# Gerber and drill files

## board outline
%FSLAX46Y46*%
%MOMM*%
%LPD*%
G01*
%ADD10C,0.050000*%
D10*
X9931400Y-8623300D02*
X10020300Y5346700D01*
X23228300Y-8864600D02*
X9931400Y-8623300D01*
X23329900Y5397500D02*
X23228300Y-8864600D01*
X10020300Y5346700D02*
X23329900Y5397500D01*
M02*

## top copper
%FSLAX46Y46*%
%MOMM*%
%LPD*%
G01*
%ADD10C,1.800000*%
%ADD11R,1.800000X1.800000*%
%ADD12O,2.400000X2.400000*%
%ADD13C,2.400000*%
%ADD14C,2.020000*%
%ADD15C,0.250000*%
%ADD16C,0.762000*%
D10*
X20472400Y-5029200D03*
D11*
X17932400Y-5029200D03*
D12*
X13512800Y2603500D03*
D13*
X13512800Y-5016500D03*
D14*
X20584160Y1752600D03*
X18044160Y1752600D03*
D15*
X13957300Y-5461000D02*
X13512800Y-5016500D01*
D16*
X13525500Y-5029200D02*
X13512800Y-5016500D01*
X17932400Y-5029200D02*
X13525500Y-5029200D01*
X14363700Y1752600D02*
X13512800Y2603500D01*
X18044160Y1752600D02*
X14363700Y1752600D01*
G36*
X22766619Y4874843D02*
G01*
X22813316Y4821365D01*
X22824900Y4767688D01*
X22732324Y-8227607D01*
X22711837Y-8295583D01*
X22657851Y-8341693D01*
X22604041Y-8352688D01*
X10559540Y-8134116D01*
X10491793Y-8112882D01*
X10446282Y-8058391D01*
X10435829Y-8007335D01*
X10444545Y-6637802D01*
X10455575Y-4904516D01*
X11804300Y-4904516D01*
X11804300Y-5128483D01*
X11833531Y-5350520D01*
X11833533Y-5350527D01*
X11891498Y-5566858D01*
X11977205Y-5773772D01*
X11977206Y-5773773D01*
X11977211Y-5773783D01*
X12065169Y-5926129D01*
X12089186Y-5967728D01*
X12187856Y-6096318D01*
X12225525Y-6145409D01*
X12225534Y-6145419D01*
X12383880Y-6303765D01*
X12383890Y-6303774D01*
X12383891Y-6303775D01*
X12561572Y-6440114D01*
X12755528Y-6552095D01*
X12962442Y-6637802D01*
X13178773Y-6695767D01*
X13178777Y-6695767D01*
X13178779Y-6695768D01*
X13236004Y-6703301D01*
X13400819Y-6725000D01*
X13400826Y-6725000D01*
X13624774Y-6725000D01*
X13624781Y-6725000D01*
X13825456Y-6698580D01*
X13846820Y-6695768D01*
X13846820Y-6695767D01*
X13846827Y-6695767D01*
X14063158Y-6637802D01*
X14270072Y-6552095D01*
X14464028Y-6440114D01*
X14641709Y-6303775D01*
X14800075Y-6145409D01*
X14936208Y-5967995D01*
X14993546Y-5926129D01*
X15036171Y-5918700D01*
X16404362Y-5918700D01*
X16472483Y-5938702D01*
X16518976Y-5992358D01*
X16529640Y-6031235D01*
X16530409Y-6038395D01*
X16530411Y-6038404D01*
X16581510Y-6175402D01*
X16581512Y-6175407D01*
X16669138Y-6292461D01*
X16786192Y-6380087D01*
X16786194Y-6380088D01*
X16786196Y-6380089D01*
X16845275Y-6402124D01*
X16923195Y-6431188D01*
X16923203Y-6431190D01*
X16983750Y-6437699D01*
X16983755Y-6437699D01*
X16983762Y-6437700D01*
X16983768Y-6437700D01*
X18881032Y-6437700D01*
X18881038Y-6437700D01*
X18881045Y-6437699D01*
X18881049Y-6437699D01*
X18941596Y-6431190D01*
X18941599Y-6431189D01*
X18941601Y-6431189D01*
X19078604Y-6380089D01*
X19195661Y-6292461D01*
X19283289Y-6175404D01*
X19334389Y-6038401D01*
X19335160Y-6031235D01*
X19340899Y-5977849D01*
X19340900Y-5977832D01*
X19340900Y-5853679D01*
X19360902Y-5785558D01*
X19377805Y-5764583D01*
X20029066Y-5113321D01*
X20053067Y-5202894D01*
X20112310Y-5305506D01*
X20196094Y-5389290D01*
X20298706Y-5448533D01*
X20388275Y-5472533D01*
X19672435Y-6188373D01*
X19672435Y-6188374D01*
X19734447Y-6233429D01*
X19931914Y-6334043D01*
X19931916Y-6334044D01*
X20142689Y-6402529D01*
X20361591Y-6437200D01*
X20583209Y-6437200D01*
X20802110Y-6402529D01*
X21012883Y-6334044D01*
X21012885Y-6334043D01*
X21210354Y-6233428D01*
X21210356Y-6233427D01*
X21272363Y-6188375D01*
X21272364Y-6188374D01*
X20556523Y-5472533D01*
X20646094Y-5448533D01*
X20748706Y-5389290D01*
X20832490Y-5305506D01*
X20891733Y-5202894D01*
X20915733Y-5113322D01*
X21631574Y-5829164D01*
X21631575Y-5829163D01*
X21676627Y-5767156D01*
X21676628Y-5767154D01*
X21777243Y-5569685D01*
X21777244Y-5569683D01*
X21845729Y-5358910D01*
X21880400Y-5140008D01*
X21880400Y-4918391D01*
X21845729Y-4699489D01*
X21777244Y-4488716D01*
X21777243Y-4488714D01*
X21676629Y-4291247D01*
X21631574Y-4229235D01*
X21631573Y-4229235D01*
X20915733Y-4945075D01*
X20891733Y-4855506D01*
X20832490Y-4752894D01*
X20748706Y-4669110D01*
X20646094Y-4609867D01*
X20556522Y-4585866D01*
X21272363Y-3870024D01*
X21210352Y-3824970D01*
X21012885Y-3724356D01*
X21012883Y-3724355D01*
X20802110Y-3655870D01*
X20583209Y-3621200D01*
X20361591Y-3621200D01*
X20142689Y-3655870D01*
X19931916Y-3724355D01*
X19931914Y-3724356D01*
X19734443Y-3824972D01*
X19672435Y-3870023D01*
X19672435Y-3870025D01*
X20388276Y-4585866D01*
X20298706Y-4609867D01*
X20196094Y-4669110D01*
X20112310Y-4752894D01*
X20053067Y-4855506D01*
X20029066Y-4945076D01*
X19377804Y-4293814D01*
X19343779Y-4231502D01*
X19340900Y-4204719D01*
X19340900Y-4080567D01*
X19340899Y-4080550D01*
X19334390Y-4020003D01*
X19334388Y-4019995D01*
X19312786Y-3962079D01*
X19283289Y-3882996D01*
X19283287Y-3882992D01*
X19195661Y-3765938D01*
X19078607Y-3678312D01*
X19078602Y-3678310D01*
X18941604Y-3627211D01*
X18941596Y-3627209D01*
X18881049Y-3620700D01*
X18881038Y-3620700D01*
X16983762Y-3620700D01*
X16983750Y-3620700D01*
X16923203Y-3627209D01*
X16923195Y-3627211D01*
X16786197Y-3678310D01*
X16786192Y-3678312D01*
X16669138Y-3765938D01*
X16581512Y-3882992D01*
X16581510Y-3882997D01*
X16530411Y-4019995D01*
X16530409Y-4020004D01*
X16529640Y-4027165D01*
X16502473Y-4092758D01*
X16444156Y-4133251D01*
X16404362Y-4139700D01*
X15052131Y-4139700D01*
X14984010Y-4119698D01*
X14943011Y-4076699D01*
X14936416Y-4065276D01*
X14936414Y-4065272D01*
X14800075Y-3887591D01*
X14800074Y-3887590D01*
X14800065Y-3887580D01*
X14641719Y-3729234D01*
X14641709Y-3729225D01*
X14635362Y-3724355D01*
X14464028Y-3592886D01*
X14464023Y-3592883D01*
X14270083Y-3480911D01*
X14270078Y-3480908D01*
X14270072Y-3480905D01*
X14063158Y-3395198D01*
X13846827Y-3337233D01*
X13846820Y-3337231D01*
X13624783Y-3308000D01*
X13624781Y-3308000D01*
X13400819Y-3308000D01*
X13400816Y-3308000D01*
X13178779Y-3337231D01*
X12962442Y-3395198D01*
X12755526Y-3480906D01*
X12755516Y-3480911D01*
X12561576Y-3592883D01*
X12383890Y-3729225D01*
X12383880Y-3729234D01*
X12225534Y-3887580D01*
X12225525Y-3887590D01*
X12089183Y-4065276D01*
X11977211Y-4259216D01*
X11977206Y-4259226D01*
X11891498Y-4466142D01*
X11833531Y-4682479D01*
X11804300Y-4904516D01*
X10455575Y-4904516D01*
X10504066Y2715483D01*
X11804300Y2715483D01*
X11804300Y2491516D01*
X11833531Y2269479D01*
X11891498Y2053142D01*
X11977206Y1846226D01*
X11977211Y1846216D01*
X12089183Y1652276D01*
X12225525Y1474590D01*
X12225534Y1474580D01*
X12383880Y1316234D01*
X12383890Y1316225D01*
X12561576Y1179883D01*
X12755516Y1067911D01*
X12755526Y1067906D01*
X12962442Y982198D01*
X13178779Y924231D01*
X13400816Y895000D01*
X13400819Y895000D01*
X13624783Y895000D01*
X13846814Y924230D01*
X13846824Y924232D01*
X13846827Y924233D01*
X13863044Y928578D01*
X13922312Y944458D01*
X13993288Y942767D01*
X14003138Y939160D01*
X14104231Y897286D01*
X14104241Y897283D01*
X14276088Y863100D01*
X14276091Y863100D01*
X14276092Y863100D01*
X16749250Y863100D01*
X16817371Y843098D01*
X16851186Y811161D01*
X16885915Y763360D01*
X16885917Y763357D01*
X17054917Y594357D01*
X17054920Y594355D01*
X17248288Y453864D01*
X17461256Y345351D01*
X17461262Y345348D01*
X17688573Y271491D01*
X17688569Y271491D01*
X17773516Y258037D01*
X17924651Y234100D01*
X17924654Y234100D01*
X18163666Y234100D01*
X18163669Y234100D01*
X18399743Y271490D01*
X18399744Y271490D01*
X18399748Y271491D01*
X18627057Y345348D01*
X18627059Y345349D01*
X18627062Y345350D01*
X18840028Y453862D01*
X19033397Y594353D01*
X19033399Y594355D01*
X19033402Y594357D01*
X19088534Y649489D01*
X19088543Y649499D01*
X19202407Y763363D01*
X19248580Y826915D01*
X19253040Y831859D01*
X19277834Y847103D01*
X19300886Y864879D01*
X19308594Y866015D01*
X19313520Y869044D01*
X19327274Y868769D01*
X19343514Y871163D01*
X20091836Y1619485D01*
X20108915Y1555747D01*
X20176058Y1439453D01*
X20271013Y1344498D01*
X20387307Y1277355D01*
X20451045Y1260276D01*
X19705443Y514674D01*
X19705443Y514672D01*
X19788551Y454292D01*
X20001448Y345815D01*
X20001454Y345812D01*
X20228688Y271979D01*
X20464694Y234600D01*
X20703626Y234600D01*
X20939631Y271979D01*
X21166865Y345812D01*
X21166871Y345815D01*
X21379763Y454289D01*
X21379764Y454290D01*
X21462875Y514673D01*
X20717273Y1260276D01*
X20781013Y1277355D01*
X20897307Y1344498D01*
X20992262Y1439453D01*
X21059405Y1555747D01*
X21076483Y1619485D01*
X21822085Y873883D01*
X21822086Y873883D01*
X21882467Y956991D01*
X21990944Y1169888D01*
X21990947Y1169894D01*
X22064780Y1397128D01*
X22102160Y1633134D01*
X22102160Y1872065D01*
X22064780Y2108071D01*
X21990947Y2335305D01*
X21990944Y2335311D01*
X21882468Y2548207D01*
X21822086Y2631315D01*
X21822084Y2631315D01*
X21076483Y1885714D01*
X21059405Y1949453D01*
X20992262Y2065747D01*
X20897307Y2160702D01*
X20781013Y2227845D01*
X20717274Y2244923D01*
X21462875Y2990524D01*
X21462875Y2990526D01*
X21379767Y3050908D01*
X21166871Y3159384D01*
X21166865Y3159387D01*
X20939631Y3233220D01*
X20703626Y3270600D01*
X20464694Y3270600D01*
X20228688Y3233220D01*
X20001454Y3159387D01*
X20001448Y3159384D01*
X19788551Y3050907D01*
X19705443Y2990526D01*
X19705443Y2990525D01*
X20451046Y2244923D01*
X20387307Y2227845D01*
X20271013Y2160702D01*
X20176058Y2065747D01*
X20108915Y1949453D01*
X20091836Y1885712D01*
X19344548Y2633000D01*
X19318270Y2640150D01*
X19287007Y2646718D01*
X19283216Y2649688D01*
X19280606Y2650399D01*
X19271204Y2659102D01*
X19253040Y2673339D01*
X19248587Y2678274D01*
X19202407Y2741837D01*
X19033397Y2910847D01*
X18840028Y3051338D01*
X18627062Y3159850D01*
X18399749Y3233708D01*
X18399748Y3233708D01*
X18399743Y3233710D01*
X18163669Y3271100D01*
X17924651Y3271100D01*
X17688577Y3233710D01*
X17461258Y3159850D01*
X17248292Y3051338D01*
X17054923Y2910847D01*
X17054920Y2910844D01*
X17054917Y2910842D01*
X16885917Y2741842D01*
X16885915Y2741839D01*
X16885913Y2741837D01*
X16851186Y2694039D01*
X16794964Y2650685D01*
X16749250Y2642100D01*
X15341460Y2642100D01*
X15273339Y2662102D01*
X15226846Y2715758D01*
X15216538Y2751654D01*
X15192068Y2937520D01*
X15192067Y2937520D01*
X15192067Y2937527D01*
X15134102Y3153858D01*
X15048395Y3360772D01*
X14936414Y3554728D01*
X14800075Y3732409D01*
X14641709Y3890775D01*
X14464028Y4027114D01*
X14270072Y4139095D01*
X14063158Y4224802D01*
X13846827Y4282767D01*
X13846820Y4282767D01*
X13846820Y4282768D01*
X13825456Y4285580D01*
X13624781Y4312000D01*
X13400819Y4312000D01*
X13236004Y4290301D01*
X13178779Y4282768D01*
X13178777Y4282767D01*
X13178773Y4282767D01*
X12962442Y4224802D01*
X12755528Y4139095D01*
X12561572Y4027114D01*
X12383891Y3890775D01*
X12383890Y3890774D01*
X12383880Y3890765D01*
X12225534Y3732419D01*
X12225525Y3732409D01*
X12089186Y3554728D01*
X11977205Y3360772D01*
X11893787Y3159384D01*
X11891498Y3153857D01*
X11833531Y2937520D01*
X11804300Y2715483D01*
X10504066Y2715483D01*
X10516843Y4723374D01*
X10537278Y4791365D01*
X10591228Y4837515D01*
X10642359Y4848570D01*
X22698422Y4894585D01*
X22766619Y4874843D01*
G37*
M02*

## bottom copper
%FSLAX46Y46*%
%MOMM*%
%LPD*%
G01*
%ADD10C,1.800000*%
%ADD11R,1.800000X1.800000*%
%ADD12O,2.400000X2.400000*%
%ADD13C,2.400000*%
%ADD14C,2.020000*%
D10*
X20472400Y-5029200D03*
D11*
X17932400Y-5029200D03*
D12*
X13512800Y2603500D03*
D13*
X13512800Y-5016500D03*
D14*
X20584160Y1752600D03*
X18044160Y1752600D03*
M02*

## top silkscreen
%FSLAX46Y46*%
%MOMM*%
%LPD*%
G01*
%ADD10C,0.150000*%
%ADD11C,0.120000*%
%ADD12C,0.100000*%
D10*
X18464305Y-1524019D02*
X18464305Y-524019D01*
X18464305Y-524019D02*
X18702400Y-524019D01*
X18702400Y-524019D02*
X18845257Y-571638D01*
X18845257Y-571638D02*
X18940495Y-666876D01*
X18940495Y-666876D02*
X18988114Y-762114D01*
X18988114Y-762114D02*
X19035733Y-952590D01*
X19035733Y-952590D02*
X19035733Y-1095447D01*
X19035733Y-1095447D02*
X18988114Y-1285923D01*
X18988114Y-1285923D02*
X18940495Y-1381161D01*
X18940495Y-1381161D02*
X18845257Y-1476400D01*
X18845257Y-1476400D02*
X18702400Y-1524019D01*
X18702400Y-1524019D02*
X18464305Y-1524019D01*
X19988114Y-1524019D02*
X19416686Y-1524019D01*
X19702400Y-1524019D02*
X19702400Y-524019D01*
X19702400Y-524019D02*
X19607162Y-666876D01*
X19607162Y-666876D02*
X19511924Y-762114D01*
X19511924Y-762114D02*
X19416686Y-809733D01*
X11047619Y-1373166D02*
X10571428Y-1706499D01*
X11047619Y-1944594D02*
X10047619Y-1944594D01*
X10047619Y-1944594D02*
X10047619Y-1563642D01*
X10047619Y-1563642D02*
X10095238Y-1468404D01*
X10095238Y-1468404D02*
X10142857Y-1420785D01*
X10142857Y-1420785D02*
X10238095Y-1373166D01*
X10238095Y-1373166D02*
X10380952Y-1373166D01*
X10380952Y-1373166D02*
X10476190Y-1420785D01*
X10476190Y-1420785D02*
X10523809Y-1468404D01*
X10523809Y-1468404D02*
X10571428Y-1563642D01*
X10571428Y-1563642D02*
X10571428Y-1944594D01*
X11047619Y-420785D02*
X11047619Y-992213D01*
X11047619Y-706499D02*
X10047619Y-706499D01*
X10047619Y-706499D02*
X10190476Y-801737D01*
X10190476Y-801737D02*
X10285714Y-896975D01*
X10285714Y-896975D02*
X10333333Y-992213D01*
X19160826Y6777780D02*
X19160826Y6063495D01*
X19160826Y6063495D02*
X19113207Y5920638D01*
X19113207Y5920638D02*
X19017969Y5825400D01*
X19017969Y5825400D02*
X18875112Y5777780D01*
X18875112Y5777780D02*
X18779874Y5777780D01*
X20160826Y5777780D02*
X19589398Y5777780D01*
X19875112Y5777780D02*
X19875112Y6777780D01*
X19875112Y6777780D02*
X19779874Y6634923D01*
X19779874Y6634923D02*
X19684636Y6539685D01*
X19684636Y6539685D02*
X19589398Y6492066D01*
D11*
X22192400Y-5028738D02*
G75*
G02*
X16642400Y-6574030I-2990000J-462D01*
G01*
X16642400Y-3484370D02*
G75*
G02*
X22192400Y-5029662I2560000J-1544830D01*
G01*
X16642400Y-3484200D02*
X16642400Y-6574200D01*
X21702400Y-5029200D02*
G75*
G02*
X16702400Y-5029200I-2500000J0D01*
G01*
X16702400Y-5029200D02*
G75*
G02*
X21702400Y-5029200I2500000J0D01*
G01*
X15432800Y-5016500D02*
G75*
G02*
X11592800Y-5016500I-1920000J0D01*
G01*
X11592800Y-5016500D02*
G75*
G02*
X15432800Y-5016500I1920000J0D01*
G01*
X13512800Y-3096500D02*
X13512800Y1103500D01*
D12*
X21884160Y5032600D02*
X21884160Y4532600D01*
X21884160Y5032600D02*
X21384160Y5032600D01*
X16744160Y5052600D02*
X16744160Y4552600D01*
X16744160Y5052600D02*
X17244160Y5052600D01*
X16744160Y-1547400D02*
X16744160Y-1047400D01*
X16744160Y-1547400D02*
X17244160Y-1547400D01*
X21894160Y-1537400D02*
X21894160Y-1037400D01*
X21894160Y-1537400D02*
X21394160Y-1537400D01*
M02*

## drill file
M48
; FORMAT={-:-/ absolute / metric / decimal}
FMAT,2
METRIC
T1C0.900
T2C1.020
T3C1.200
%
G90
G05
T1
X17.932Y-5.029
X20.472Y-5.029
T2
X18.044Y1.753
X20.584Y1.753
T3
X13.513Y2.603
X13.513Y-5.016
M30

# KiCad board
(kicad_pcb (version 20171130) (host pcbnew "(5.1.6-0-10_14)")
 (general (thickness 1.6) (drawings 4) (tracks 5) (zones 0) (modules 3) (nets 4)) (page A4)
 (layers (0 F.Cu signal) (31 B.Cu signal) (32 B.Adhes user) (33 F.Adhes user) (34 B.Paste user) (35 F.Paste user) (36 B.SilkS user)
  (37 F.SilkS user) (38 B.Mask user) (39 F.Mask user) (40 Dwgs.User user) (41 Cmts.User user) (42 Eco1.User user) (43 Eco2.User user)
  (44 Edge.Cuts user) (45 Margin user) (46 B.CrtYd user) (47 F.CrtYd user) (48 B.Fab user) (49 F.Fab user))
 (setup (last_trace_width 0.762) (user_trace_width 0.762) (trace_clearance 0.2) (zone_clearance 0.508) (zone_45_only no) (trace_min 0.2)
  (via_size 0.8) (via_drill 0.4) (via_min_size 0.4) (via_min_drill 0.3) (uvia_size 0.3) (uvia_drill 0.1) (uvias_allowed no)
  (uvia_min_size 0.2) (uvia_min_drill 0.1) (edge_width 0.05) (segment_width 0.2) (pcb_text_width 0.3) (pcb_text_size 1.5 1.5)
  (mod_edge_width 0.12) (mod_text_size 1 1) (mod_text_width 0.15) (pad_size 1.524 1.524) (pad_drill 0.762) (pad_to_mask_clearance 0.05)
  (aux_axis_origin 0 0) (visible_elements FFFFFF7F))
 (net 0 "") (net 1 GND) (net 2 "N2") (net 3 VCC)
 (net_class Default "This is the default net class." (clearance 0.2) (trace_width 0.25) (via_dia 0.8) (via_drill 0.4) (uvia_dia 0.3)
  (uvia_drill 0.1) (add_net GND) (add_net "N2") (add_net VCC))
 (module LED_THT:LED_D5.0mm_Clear (layer F.Cu) (at 17.9324 5.0292)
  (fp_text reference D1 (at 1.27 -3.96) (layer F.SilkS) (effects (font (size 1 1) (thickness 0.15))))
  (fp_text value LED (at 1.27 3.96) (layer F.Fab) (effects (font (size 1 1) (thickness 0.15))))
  (fp_arc (start 1.27 0) (end -1.29 1.54483) (angle -148.9) (layer F.SilkS) (width 0.12))
  (fp_arc (start 1.27 0) (end -1.29 -1.54483) (angle 148.9) (layer F.SilkS) (width 0.12))
  (fp_line (start -1.29 -1.545) (end -1.29 1.545) (layer F.SilkS) (width 0.12))
  (fp_circle (center 1.27 0) (end 3.77 0) (layer F.SilkS) (width 0.12))
  (pad 2 thru_hole circle (at 2.54 0) (size 1.8 1.8) (drill 0.9) (layers *.Cu *.Mask) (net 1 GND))
  (pad 1 thru_hole rect (at 0 0) (size 1.8 1.8) (drill 0.9) (layers *.Cu *.Mask) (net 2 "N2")))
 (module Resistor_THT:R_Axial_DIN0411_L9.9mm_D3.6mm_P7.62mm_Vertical (layer F.Cu) (at 13.5128 5.0165 90)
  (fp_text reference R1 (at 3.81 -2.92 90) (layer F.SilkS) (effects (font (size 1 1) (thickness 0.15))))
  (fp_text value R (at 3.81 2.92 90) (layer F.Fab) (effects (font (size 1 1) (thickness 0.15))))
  (fp_circle (center 0 0) (end 1.92 0) (layer F.SilkS) (width 0.12))
  (fp_line (start 1.92 0) (end 6.12 0) (layer F.SilkS) (width 0.12))
  (pad 2 thru_hole oval (at 7.62 0 90) (size 2.4 2.4) (drill 1.2) (layers *.Cu *.Mask) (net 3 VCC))
  (pad 1 thru_hole circle (at 0 0 90) (size 2.4 2.4) (drill 1.2) (layers *.Cu *.Mask) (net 2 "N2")))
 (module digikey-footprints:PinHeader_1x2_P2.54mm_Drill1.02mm (layer F.Cu) (at 18.04416 -1.7526)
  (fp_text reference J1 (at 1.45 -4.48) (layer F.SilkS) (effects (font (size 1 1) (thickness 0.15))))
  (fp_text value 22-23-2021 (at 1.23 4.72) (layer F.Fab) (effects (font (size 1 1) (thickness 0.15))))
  (fp_line (start 3.84 -3.28) (end 3.84 -2.78) (layer F.SilkS) (width 0.1))
  (fp_line (start 3.84 -3.28) (end 3.34 -3.28) (layer F.SilkS) (width 0.1))
  (fp_line (start -1.3 -3.3) (end -1.3 -2.8) (layer F.SilkS) (width 0.1))
  (fp_line (start -1.3 -3.3) (end -0.8 -3.3) (layer F.SilkS) (width 0.1))
  (fp_line (start -1.3 3.3) (end -1.3 2.8) (layer F.SilkS) (width 0.1))
  (fp_line (start -1.3 3.3) (end -0.8 3.3) (layer F.SilkS) (width 0.1))
  (fp_line (start 3.85 3.29) (end 3.85 2.79) (layer F.SilkS) (width 0.1))
  (fp_line (start 3.85 3.29) (end 3.35 3.29) (layer F.SilkS) (width 0.1))
  (pad 2 thru_hole circle (at 2.54 0) (size 2.02 2.02) (drill 1.02) (layers *.Cu *.Mask) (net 1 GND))
  (pad 1 thru_hole circle (at 0 0) (size 2.02 2.02) (drill 1.02) (layers *.Cu *.Mask) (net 3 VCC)))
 (gr_line (start 9.9314 8.6233) (end 10.0203 -5.3467) (layer Edge.Cuts) (width 0.05))
 (gr_line (start 23.2283 8.8646) (end 9.9314 8.6233) (layer Edge.Cuts) (width 0.05))
 (gr_line (start 23.3299 -5.3975) (end 23.2283 8.8646) (layer Edge.Cuts) (width 0.05))
 (gr_line (start 10.0203 -5.3467) (end 23.3299 -5.3975) (layer Edge.Cuts) (width 0.05))
 (segment (start 13.9573 5.461) (end 13.5128 5.0165) (width 0.25) (layer F.Cu) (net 2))
 (segment (start 13.5255 5.0292) (end 13.5128 5.0165) (width 0.762) (layer F.Cu) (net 2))
 (segment (start 17.9324 5.0292) (end 13.5255 5.0292) (width 0.762) (layer F.Cu) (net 2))
 (segment (start 14.3637 -1.7526) (end 13.5128 -2.6035) (width 0.762) (layer F.Cu) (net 3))
 (segment (start 18.04416 -1.7526) (end 14.3637 -1.7526) (width 0.762) (layer F.Cu) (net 3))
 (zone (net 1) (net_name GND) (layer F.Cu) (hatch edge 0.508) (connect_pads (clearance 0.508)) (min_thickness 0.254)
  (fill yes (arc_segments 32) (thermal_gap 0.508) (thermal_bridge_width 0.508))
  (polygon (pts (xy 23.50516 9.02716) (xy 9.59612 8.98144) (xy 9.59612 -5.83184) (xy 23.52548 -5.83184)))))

